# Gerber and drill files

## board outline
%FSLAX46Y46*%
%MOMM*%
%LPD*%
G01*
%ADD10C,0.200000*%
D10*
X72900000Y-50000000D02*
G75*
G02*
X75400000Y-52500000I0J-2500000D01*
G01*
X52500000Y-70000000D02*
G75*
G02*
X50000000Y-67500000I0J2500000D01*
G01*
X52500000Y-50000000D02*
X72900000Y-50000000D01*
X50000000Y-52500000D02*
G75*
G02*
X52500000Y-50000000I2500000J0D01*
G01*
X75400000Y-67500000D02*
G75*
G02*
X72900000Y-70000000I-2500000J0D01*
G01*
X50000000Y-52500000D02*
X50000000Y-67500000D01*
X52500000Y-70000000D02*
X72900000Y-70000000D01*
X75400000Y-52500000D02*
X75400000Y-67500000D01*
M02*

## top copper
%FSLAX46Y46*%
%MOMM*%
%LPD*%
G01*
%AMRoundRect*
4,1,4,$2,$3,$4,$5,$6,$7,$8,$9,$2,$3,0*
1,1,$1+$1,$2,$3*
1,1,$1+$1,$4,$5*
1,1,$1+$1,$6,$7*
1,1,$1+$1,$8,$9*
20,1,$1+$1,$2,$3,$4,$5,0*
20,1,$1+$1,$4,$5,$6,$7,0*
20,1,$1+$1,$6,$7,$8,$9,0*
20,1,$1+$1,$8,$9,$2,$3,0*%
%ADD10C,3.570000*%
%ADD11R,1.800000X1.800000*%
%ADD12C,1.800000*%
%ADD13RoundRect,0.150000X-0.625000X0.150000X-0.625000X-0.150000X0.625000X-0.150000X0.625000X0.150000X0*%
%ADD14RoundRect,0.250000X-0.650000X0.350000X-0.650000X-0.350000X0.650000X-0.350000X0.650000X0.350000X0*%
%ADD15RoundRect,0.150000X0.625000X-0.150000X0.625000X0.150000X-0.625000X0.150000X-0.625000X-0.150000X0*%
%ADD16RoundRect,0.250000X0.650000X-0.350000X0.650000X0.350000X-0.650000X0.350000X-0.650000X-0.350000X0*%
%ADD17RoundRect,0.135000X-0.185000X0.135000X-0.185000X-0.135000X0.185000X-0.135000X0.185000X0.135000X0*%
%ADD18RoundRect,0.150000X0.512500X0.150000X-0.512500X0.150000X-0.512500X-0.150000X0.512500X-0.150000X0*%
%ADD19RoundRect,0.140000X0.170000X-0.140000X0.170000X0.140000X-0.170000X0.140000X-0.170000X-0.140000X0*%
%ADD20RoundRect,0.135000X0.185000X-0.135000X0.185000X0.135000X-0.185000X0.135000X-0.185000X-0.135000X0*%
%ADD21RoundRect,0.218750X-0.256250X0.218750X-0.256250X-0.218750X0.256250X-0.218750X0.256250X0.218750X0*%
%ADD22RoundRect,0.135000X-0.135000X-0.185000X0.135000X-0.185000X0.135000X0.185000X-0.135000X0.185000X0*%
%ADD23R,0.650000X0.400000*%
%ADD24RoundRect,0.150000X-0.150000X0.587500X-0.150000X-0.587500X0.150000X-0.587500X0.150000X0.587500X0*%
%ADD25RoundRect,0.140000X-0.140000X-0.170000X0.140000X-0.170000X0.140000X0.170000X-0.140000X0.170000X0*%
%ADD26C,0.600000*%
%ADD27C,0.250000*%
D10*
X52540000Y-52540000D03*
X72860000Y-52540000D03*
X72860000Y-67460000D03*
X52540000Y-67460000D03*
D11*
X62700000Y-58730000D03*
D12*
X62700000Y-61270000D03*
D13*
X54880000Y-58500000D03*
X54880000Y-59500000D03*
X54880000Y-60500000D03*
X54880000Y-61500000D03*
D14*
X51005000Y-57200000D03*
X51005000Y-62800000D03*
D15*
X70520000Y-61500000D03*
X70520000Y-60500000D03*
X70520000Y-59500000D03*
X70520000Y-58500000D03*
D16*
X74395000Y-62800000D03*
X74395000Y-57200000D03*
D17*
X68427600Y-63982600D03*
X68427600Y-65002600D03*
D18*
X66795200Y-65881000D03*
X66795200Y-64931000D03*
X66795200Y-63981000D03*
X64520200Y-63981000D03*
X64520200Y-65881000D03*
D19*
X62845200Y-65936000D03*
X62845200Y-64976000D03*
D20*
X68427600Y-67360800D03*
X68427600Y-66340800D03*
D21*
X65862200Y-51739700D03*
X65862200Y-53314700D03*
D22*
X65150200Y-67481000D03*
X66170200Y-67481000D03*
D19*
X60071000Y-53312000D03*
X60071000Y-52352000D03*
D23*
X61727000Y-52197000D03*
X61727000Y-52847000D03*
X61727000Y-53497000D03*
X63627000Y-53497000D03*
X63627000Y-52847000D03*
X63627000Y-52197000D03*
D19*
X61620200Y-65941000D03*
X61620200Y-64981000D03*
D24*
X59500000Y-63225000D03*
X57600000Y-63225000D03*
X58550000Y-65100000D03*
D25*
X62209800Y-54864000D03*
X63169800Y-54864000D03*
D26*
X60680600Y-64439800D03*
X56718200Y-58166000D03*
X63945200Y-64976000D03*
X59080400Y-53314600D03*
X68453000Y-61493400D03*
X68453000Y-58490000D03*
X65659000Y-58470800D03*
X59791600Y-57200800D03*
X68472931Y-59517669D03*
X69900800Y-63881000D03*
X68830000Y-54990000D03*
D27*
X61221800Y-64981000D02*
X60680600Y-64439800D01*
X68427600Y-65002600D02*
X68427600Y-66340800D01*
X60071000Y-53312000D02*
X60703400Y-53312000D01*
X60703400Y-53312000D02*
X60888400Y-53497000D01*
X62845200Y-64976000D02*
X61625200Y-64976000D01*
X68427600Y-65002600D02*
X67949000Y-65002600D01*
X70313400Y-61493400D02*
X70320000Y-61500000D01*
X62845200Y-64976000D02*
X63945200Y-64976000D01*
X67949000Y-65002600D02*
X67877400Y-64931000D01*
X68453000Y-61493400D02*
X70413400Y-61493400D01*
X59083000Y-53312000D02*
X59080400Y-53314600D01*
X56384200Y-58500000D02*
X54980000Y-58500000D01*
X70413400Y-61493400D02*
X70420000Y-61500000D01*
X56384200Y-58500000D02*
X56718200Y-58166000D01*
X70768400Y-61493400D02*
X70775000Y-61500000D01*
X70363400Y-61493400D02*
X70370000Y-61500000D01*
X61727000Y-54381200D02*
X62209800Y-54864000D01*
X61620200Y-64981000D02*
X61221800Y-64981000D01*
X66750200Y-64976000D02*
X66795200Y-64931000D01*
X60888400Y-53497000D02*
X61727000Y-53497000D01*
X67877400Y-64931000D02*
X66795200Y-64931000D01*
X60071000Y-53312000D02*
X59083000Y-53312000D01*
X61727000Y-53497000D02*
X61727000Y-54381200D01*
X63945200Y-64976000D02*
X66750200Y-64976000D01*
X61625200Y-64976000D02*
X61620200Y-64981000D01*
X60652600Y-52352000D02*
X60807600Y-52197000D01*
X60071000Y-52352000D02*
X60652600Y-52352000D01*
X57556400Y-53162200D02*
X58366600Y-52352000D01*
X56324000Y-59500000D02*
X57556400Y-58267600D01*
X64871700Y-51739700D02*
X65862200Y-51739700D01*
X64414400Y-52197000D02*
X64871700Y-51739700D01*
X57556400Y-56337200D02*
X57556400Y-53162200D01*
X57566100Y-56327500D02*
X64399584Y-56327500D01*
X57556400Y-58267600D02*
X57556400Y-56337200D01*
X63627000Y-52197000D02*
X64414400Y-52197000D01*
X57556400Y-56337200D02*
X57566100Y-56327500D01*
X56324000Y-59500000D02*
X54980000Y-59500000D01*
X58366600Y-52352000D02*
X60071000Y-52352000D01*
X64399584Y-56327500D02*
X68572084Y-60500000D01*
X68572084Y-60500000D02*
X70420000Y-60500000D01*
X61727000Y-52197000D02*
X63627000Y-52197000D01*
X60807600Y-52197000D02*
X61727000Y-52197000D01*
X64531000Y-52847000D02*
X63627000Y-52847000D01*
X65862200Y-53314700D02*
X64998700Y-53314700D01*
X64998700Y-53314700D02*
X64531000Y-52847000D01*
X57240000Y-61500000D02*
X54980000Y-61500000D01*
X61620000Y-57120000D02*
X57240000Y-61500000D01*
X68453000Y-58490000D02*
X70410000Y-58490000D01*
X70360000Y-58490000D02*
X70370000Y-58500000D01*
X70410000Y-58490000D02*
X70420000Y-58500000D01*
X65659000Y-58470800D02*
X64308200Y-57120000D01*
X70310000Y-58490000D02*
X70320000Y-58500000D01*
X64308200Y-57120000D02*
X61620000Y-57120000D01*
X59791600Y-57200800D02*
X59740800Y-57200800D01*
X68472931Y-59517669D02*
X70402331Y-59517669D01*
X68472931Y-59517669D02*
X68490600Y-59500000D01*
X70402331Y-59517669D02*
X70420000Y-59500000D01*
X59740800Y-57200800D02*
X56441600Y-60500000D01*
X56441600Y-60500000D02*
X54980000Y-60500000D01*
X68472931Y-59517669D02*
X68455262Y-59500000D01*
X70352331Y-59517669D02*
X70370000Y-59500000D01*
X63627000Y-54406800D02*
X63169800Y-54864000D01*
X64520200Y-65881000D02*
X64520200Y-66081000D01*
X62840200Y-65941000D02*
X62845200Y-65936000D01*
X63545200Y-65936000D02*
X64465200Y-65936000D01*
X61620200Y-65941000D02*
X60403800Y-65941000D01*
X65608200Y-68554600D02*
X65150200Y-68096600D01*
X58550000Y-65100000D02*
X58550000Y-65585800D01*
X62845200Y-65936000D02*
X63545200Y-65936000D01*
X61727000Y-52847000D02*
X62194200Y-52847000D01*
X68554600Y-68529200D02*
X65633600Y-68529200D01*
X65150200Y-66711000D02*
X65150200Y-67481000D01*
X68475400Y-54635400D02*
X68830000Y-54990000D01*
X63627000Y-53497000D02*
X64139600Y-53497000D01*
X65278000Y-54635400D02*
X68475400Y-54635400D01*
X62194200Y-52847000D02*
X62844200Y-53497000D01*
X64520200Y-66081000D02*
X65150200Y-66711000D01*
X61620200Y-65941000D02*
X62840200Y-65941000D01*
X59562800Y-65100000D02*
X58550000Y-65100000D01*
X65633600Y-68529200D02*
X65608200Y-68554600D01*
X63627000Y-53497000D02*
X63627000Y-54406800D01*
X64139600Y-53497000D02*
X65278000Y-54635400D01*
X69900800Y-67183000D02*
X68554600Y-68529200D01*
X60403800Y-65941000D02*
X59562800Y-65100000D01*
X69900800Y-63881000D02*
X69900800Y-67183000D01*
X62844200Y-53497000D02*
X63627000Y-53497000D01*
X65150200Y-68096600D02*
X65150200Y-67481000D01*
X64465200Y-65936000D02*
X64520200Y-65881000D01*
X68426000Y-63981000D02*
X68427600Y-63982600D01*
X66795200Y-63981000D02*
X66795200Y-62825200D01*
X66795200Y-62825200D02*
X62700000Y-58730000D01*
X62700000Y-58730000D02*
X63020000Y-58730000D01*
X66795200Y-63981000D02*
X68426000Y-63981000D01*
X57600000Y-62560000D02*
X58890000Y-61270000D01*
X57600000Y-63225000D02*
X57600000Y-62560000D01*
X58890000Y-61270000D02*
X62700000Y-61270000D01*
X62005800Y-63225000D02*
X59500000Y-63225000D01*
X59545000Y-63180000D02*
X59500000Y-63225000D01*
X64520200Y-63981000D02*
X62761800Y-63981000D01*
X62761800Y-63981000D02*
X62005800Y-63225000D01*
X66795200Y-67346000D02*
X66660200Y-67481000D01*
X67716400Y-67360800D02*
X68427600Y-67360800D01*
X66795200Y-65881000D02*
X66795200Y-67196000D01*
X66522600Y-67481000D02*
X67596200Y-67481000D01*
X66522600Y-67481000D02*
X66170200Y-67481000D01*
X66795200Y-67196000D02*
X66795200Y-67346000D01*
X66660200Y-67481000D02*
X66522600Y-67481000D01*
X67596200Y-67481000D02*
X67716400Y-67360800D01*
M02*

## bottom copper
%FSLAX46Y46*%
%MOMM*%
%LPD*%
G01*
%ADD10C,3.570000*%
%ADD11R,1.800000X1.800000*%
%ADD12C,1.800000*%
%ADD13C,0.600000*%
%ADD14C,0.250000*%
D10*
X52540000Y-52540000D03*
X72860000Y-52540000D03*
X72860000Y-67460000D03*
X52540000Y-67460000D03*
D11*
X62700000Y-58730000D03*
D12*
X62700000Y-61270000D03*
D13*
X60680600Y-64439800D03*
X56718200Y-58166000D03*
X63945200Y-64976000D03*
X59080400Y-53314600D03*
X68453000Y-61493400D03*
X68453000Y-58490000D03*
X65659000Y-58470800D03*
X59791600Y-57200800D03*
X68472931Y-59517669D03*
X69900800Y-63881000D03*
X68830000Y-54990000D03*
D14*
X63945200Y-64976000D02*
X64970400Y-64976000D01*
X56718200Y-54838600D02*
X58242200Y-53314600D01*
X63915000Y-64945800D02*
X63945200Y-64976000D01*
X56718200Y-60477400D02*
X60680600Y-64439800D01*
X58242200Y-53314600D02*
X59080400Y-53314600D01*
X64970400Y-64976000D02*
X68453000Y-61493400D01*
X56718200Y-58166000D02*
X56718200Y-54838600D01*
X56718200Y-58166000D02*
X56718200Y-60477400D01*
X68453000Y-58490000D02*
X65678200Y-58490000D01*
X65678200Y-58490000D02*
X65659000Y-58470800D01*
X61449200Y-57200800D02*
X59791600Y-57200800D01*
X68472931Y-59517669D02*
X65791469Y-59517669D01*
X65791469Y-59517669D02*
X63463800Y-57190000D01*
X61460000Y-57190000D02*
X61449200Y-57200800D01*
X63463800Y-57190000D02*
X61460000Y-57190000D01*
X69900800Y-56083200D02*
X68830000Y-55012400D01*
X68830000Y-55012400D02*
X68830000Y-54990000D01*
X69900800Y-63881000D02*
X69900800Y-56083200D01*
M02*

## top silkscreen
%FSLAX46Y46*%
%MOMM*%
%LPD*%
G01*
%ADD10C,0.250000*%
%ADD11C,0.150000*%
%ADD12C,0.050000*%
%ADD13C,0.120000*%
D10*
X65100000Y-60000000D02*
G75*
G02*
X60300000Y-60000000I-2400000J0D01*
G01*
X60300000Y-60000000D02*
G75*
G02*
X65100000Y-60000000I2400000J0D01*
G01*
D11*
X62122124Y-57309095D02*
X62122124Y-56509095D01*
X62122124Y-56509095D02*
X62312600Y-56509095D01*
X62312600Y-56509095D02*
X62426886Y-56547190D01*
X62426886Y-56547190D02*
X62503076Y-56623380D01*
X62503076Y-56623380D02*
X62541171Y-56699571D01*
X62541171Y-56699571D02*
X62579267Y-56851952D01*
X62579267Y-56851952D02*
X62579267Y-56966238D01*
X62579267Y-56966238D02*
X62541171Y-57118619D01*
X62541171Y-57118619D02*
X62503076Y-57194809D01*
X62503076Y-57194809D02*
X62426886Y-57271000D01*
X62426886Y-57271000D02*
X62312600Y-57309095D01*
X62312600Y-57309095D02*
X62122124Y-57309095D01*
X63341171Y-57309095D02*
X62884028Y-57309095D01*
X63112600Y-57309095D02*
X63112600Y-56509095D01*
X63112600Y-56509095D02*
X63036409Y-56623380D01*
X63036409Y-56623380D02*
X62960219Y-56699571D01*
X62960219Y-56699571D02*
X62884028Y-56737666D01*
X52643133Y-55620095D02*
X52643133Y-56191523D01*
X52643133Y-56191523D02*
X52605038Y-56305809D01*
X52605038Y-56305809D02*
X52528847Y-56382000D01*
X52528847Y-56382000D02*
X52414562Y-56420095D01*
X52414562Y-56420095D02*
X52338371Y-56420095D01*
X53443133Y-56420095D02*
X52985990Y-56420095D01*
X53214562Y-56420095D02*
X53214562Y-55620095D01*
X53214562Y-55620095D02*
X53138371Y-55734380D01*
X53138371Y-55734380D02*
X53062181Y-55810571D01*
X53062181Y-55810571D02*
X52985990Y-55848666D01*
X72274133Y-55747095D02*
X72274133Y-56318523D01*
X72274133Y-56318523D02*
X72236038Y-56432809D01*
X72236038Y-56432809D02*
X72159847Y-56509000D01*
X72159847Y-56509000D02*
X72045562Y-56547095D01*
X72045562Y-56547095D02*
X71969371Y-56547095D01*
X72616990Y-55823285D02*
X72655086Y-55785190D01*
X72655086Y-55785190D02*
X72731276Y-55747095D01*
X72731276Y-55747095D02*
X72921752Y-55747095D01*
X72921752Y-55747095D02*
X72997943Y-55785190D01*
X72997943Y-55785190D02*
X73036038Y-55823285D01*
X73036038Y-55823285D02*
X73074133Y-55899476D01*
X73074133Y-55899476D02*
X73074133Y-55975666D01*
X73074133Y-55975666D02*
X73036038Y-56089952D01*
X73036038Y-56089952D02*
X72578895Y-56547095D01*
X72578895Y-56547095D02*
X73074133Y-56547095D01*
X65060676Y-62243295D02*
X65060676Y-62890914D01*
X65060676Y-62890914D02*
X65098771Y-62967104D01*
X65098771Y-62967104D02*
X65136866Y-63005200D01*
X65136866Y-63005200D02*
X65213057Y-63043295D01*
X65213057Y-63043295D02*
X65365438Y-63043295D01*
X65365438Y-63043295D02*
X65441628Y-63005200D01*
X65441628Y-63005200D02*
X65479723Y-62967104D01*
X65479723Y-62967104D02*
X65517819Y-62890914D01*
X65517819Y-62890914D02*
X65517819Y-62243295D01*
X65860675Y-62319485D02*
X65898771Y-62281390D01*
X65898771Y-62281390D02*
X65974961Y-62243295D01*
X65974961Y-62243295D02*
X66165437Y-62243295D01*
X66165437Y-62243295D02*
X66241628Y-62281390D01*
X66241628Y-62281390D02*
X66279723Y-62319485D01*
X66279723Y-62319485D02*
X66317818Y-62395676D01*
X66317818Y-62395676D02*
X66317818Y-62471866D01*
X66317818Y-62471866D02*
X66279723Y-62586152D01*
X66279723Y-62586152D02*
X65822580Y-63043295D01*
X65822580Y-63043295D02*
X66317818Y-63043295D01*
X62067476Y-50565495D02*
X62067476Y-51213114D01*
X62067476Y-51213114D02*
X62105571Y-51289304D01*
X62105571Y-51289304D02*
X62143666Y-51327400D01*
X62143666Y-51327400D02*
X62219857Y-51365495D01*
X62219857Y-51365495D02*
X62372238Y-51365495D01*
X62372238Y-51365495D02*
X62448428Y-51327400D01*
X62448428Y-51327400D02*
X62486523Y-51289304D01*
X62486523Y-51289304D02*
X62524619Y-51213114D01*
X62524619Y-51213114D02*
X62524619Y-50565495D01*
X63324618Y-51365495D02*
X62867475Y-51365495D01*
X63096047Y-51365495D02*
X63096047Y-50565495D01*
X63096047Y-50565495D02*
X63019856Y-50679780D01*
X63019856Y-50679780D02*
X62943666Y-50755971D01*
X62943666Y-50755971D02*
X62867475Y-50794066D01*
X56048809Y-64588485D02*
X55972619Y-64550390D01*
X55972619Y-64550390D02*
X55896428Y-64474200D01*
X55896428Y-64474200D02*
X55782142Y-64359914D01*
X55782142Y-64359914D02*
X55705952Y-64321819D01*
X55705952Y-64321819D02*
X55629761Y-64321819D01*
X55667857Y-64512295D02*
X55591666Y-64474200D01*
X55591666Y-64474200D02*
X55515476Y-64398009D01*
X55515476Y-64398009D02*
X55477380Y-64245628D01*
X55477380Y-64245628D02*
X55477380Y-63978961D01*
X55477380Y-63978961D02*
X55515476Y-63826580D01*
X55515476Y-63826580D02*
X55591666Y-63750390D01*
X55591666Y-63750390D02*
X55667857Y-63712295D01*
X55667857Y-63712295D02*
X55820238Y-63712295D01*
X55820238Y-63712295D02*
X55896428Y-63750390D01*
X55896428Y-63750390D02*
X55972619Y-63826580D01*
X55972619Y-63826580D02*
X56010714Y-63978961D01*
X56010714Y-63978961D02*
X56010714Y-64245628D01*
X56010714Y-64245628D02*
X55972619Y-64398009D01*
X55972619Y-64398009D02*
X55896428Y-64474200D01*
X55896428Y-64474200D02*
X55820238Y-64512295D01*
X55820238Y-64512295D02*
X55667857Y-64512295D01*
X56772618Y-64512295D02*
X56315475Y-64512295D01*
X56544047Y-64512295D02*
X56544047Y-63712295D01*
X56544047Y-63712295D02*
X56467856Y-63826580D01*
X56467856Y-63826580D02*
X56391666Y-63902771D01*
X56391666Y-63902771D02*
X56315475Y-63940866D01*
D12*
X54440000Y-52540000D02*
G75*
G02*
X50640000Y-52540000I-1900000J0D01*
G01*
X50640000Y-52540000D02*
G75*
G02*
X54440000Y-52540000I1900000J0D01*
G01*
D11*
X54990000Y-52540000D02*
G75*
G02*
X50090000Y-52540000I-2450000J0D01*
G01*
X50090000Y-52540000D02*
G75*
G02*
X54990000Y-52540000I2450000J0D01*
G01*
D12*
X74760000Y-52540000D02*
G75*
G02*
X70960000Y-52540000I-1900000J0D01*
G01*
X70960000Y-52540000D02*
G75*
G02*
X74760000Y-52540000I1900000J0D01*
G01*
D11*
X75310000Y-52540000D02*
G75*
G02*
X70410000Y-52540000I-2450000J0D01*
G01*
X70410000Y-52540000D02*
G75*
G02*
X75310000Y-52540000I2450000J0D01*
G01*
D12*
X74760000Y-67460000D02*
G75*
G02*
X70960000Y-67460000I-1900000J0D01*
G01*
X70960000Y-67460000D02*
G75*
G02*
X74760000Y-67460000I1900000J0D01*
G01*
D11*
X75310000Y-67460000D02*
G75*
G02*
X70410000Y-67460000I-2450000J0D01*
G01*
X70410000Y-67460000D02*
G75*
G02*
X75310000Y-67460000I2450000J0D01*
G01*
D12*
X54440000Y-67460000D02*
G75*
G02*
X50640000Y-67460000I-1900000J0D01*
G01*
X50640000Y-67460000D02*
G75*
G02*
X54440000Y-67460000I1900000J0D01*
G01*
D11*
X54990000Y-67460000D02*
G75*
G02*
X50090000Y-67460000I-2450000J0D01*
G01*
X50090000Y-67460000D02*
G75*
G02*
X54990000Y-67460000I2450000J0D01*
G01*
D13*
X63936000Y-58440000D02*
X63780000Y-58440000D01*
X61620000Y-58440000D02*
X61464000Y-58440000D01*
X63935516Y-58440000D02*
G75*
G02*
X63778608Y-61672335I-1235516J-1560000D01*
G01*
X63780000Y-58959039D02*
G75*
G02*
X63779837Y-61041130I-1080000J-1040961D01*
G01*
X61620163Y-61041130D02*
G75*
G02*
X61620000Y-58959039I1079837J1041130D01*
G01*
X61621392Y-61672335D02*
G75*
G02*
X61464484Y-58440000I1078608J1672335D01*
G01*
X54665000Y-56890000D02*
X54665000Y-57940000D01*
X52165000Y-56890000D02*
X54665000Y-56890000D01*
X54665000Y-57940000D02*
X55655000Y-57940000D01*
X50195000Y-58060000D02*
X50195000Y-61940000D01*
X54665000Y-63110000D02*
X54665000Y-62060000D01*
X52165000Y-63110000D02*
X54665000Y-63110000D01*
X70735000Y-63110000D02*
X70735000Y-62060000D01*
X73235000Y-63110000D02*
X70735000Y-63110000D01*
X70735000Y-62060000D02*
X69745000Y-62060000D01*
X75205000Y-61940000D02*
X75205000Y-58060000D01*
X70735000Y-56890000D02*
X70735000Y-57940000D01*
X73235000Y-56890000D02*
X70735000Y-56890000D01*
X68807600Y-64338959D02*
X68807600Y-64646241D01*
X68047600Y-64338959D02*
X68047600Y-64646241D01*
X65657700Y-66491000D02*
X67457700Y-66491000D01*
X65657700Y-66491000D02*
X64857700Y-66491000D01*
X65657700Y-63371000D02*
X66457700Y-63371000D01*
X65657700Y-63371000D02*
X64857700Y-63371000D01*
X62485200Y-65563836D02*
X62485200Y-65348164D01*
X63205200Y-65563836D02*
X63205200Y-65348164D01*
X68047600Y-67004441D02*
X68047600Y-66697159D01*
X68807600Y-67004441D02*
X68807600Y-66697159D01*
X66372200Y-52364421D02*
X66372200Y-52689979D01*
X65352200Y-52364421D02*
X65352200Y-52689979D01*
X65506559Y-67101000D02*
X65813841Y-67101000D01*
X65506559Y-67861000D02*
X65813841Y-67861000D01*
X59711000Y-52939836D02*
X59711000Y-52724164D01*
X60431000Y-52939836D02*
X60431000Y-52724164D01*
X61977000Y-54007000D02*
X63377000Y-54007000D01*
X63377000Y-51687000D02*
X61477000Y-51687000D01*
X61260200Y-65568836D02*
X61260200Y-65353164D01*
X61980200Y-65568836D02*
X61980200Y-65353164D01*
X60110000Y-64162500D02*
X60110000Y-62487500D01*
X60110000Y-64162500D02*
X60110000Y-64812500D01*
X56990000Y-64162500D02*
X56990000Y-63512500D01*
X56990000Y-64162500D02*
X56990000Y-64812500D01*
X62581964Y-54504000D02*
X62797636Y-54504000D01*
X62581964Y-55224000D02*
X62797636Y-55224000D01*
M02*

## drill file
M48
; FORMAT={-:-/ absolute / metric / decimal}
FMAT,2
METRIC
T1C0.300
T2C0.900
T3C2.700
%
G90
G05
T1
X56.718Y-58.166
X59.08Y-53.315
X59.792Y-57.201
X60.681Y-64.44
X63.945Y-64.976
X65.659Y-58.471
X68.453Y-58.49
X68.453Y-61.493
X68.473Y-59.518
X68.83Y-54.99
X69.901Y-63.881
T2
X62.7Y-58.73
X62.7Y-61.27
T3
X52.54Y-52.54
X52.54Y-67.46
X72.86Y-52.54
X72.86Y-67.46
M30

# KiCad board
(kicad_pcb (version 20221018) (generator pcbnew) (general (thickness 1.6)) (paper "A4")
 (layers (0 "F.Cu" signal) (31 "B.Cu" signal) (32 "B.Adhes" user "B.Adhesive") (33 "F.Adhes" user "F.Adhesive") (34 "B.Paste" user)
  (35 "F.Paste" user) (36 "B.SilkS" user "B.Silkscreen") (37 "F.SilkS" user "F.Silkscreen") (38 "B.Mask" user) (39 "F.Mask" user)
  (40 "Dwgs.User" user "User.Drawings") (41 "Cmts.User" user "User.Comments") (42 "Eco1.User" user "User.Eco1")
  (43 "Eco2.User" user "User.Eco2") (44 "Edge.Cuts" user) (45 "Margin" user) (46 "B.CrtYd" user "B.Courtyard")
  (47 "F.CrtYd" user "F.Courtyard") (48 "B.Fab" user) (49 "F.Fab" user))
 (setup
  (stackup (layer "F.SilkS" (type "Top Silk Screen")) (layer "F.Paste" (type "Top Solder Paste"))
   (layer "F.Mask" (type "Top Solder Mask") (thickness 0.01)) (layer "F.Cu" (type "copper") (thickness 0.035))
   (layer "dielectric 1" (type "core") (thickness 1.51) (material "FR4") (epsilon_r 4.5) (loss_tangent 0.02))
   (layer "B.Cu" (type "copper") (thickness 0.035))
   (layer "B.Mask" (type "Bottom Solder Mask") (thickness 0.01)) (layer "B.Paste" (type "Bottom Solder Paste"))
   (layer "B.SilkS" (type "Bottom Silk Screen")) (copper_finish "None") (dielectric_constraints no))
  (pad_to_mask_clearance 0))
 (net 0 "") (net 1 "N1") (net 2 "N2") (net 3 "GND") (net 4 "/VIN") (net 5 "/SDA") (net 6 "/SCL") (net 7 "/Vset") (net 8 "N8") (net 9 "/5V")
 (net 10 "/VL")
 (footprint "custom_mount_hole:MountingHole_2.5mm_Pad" (layer "F.Cu") (at 52.54 52.54)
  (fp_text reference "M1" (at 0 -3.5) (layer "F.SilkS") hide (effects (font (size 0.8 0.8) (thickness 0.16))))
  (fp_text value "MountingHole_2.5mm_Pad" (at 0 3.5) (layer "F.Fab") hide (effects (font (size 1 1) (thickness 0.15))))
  (fp_circle (center 0 0) (end 1.9 0) (stroke (width 0.05) (type solid)) (fill none) (layer "F.SilkS"))
  (fp_circle (center 0 0) (end 2.45 0) (stroke (width 0.15) (type solid)) (fill none) (layer "F.SilkS"))
  (pad "~" thru_hole circle (at 0 0) (size 3.57 3.57) (drill 2.7) (layers "*.Cu" "*.Mask")))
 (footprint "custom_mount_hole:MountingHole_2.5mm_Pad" (layer "F.Cu") (at 72.86 52.54)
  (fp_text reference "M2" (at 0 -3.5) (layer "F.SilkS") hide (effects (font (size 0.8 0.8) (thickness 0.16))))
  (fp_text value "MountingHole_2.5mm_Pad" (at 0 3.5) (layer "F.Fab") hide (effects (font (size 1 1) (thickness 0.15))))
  (fp_circle (center 0 0) (end 1.9 0) (stroke (width 0.05) (type solid)) (fill none) (layer "F.SilkS"))
  (fp_circle (center 0 0) (end 2.45 0) (stroke (width 0.15) (type solid)) (fill none) (layer "F.SilkS"))
  (pad "~" thru_hole circle (at 0 0) (size 3.57 3.57) (drill 2.7) (layers "*.Cu" "*.Mask")))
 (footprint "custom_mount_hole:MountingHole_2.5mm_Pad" (layer "F.Cu") (at 72.86 67.46)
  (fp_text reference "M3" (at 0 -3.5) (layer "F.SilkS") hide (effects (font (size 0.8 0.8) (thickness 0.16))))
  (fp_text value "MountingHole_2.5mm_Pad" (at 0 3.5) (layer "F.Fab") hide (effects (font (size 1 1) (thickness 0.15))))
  (fp_circle (center 0 0) (end 1.9 0) (stroke (width 0.05) (type solid)) (fill none) (layer "F.SilkS"))
  (fp_circle (center 0 0) (end 2.45 0) (stroke (width 0.15) (type solid)) (fill none) (layer "F.SilkS"))
  (pad "~" thru_hole circle (at 0 0) (size 3.57 3.57) (drill 2.7) (layers "*.Cu" "*.Mask")))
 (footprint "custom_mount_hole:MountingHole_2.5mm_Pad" (layer "F.Cu") (at 52.54 67.46)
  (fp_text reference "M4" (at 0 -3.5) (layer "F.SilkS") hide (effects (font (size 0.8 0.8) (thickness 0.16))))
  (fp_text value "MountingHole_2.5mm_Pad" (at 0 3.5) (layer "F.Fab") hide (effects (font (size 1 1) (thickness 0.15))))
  (fp_circle (center 0 0) (end 1.9 0) (stroke (width 0.05) (type solid)) (fill none) (layer "F.SilkS"))
  (fp_circle (center 0 0) (end 2.45 0) (stroke (width 0.15) (type solid)) (fill none) (layer "F.SilkS"))
  (pad "~" thru_hole circle (at 0 0) (size 3.57 3.57) (drill 2.7) (layers "*.Cu" "*.Mask")))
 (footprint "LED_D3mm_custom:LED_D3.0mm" (layer "F.Cu") (at 62.7 58.73 -90)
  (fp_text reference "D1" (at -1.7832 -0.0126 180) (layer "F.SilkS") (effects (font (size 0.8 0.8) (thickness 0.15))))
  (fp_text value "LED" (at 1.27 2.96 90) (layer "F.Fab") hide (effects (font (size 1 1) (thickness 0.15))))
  (fp_line (start -0.29 -1.236) (end -0.29 -1.08) (stroke (width 0.12) (type solid)) (layer "F.SilkS"))
  (fp_line (start -0.29 1.08) (end -0.29 1.236) (stroke (width 0.12) (type solid)) (layer "F.SilkS"))
  (fp_arc (start -0.29 -1.235516) (mid 1.366487 -1.987659) (end 2.942335 -1.078608) (stroke (width 0.12) (type solid)) (layer "F.SilkS"))
  (fp_arc (start 0.229039 -1.08) (mid 1.270117 -1.5) (end 2.31113 -1.079837) (stroke (width 0.12) (type solid)) (layer "F.SilkS"))
  (fp_arc (start 2.31113 1.079837) (mid 1.270117 1.5) (end 0.229039 1.08) (stroke (width 0.12) (type solid)) (layer "F.SilkS"))
  (fp_arc (start 2.942335 1.078608) (mid 1.366487 1.987659) (end -0.29 1.235516) (stroke (width 0.12) (type solid)) (layer "F.SilkS"))
  (pad "1" thru_hole rect (at 0 0 270) (size 1.8 1.8) (drill 0.9) (layers "*.Cu" "*.Mask") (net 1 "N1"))
  (pad "2" thru_hole circle (at 2.54 0 270) (size 1.8 1.8) (drill 0.9) (layers "*.Cu" "*.Mask") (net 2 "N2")))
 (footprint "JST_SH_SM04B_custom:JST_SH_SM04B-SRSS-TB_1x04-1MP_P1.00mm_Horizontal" (layer "F.Cu") (at 52.88 60 -90)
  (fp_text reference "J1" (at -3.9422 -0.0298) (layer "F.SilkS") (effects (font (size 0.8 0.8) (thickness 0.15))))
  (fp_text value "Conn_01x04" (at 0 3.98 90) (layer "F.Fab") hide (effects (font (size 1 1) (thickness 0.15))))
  (fp_line (start -3.11 -1.785) (end -2.06 -1.785) (stroke (width 0.12) (type solid)) (layer "F.SilkS"))
  (fp_line (start -3.11 0.715) (end -3.11 -1.785) (stroke (width 0.12) (type solid)) (layer "F.SilkS"))
  (fp_line (start -2.06 -1.785) (end -2.06 -2.775) (stroke (width 0.12) (type solid)) (layer "F.SilkS"))
  (fp_line (start -1.94 2.685) (end 1.94 2.685) (stroke (width 0.12) (type solid)) (layer "F.SilkS"))
  (fp_line (start 3.11 -1.785) (end 2.06 -1.785) (stroke (width 0.12) (type solid)) (layer "F.SilkS"))
  (fp_line (start 3.11 0.715) (end 3.11 -1.785) (stroke (width 0.12) (type solid)) (layer "F.SilkS"))
  (pad "1" smd roundrect (at -1.5 -2 270) (size 0.6 1.55) (layers "F.Cu" "F.Paste" "F.Mask") (roundrect_rratio 0.25) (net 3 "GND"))
  (pad "2" smd roundrect (at -0.5 -2 270) (size 0.6 1.55) (layers "F.Cu" "F.Paste" "F.Mask") (roundrect_rratio 0.25) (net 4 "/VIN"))
  (pad "3" smd roundrect (at 0.5 -2 270) (size 0.6 1.55) (layers "F.Cu" "F.Paste" "F.Mask") (roundrect_rratio 0.25) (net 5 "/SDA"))
  (pad "4" smd roundrect (at 1.5 -2 270) (size 0.6 1.55) (layers "F.Cu" "F.Paste" "F.Mask") (roundrect_rratio 0.25) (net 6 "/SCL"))
  (pad "MP" smd roundrect (at -2.8 1.875 270) (size 1.2 1.8) (layers "F.Cu" "F.Paste" "F.Mask") (roundrect_rratio 0.2083333333))
  (pad "MP" smd roundrect (at 2.8 1.875 270) (size 1.2 1.8) (layers "F.Cu" "F.Paste" "F.Mask") (roundrect_rratio 0.2083333333)))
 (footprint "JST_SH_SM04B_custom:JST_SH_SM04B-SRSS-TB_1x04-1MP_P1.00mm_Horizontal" (layer "F.Cu") (at 72.52 60 90)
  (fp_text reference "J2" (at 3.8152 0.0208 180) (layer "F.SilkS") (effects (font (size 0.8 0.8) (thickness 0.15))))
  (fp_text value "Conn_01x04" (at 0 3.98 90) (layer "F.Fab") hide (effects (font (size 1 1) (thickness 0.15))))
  (fp_line (start -3.11 -1.785) (end -2.06 -1.785) (stroke (width 0.12) (type solid)) (layer "F.SilkS"))
  (fp_line (start -3.11 0.715) (end -3.11 -1.785) (stroke (width 0.12) (type solid)) (layer "F.SilkS"))
  (fp_line (start -2.06 -1.785) (end -2.06 -2.775) (stroke (width 0.12) (type solid)) (layer "F.SilkS"))
  (fp_line (start -1.94 2.685) (end 1.94 2.685) (stroke (width 0.12) (type solid)) (layer "F.SilkS"))
  (fp_line (start 3.11 -1.785) (end 2.06 -1.785) (stroke (width 0.12) (type solid)) (layer "F.SilkS"))
  (fp_line (start 3.11 0.715) (end 3.11 -1.785) (stroke (width 0.12) (type solid)) (layer "F.SilkS"))
  (pad "1" smd roundrect (at -1.5 -2 90) (size 0.6 1.55) (layers "F.Cu" "F.Paste" "F.Mask") (roundrect_rratio 0.25) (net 3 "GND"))
  (pad "2" smd roundrect (at -0.5 -2 90) (size 0.6 1.55) (layers "F.Cu" "F.Paste" "F.Mask") (roundrect_rratio 0.25) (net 4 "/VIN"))
  (pad "3" smd roundrect (at 0.5 -2 90) (size 0.6 1.55) (layers "F.Cu" "F.Paste" "F.Mask") (roundrect_rratio 0.25) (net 5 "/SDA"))
  (pad "4" smd roundrect (at 1.5 -2 90) (size 0.6 1.55) (layers "F.Cu" "F.Paste" "F.Mask") (roundrect_rratio 0.25) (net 6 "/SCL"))
  (pad "MP" smd roundrect (at -2.8 1.875 90) (size 1.2 1.8) (layers "F.Cu" "F.Paste" "F.Mask") (roundrect_rratio 0.2083333333))
  (pad "MP" smd roundrect (at 2.8 1.875 90) (size 1.2 1.8) (layers "F.Cu" "F.Paste" "F.Mask") (roundrect_rratio 0.2083333333)))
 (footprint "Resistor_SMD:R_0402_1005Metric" (layer "F.Cu") (at 68.4276 64.4926 -90)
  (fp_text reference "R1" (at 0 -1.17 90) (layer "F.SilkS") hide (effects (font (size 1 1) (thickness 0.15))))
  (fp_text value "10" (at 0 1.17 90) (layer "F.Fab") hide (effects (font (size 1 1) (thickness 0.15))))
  (fp_line (start -0.153641 -0.38) (end 0.153641 -0.38) (stroke (width 0.12) (type solid)) (layer "F.SilkS"))
  (fp_line (start -0.153641 0.38) (end 0.153641 0.38) (stroke (width 0.12) (type solid)) (layer "F.SilkS"))
  (pad "1" smd roundrect (at -0.51 0 270) (size 0.54 0.64) (layers "F.Cu" "F.Paste" "F.Mask") (roundrect_rratio 0.25) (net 1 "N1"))
  (pad "2" smd roundrect (at 0.51 0 270) (size 0.54 0.64) (layers "F.Cu" "F.Paste" "F.Mask") (roundrect_rratio 0.25) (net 3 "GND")))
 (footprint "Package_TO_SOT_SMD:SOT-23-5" (layer "F.Cu") (at 65.6577 64.931 180)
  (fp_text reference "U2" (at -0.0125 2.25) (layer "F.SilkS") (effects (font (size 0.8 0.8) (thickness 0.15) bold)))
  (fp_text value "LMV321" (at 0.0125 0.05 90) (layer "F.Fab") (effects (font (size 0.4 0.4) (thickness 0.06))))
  (fp_line (start 0 -1.56) (end -1.8 -1.56) (stroke (width 0.12) (type solid)) (layer "F.SilkS"))
  (fp_line (start 0 -1.56) (end 0.8 -1.56) (stroke (width 0.12) (type solid)) (layer "F.SilkS"))
  (fp_line (start 0 1.56) (end -0.8 1.56) (stroke (width 0.12) (type solid)) (layer "F.SilkS"))
  (fp_line (start 0 1.56) (end 0.8 1.56) (stroke (width 0.12) (type solid)) (layer "F.SilkS"))
  (pad "1" smd roundrect (at -1.1375 -0.95 180) (size 1.325 0.6) (layers "F.Cu" "F.Paste" "F.Mask") (roundrect_rratio 0.25) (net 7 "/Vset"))
  (pad "2" smd roundrect (at -1.1375 0 180) (size 1.325 0.6) (layers "F.Cu" "F.Paste" "F.Mask") (roundrect_rratio 0.25) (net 3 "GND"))
  (pad "3" smd roundrect (at -1.1375 0.95 180) (size 1.325 0.6) (layers "F.Cu" "F.Paste" "F.Mask") (roundrect_rratio 0.25) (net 1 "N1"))
  (pad "4" smd roundrect (at 1.1375 0.95 180) (size 1.325 0.6) (layers "F.Cu" "F.Paste" "F.Mask") (roundrect_rratio 0.25) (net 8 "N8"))
  (pad "5" smd roundrect (at 1.1375 -0.95 180) (size 1.325 0.6) (layers "F.Cu" "F.Paste" "F.Mask") (roundrect_rratio 0.25) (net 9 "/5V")))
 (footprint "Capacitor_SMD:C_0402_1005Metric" (layer "F.Cu") (at 62.8452 65.456 90)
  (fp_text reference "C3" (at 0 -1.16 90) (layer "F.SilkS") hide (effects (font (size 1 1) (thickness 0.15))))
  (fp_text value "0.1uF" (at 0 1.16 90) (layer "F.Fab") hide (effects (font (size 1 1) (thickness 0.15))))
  (fp_line (start -0.107836 -0.36) (end 0.107836 -0.36) (stroke (width 0.12) (type solid)) (layer "F.SilkS"))
  (fp_line (start -0.107836 0.36) (end 0.107836 0.36) (stroke (width 0.12) (type solid)) (layer "F.SilkS"))
  (pad "1" smd roundrect (at -0.48 0 90) (size 0.56 0.62) (layers "F.Cu" "F.Paste" "F.Mask") (roundrect_rratio 0.25) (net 9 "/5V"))
  (pad "2" smd roundrect (at 0.48 0 90) (size 0.56 0.62) (layers "F.Cu" "F.Paste" "F.Mask") (roundrect_rratio 0.25) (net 3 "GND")))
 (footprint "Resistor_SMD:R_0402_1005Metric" (layer "F.Cu") (at 68.4276 66.8508 90)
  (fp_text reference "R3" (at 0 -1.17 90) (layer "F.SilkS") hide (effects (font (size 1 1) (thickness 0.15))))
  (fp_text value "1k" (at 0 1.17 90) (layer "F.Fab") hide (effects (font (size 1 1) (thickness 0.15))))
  (fp_line (start -0.153641 -0.38) (end 0.153641 -0.38) (stroke (width 0.12) (type solid)) (layer "F.SilkS"))
  (fp_line (start -0.153641 0.38) (end 0.153641 0.38) (stroke (width 0.12) (type solid)) (layer "F.SilkS"))
  (pad "1" smd roundrect (at -0.51 0 90) (size 0.54 0.64) (layers "F.Cu" "F.Paste" "F.Mask") (roundrect_rratio 0.25) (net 7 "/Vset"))
  (pad "2" smd roundrect (at 0.51 0 90) (size 0.54 0.64) (layers "F.Cu" "F.Paste" "F.Mask") (roundrect_rratio 0.25) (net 3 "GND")))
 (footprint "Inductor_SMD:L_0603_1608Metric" (layer "F.Cu") (at 65.8622 52.5272 -90)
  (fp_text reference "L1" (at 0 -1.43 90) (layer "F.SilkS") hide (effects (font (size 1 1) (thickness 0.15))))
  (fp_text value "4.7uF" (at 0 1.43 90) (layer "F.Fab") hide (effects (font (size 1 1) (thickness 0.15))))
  (fp_line (start -0.162779 -0.51) (end 0.162779 -0.51) (stroke (width 0.12) (type solid)) (layer "F.SilkS"))
  (fp_line (start -0.162779 0.51) (end 0.162779 0.51) (stroke (width 0.12) (type solid)) (layer "F.SilkS"))
  (pad "1" smd roundrect (at -0.7875 0 270) (size 0.875 0.95) (layers "F.Cu" "F.Paste" "F.Mask") (roundrect_rratio 0.25) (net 4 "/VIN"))
  (pad "2" smd roundrect (at 0.7875 0 270) (size 0.875 0.95) (layers "F.Cu" "F.Paste" "F.Mask") (roundrect_rratio 0.25) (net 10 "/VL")))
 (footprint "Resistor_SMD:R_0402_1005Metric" (layer "F.Cu") (at 65.6602 67.481)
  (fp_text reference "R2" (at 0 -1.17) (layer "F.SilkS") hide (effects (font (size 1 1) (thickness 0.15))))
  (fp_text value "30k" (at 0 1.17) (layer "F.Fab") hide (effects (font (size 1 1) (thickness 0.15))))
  (fp_line (start -0.153641 -0.38) (end 0.153641 -0.38) (stroke (width 0.12) (type solid)) (layer "F.SilkS"))
  (fp_line (start -0.153641 0.38) (end 0.153641 0.38) (stroke (width 0.12) (type solid)) (layer "F.SilkS"))
  (pad "1" smd roundrect (at -0.51 0) (size 0.54 0.64) (layers "F.Cu" "F.Paste" "F.Mask") (roundrect_rratio 0.25) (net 9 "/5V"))
  (pad "2" smd roundrect (at 0.51 0) (size 0.54 0.64) (layers "F.Cu" "F.Paste" "F.Mask") (roundrect_rratio 0.25) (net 7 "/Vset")))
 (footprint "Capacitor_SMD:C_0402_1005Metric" (layer "F.Cu") (at 60.071 52.832 90)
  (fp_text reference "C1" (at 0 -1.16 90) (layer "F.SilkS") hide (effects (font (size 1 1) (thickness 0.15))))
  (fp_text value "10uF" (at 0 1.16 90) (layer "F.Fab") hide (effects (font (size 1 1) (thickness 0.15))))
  (fp_line (start -0.107836 -0.36) (end 0.107836 -0.36) (stroke (width 0.12) (type solid)) (layer "F.SilkS"))
  (fp_line (start -0.107836 0.36) (end 0.107836 0.36) (stroke (width 0.12) (type solid)) (layer "F.SilkS"))
  (pad "1" smd roundrect (at -0.48 0 90) (size 0.56 0.62) (layers "F.Cu" "F.Paste" "F.Mask") (roundrect_rratio 0.25) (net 3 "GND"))
  (pad "2" smd roundrect (at 0.48 0 90) (size 0.56 0.62) (layers "F.Cu" "F.Paste" "F.Mask") (roundrect_rratio 0.25) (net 4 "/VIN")))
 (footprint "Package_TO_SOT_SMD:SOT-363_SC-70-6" (layer "F.Cu") (at 62.677 52.847)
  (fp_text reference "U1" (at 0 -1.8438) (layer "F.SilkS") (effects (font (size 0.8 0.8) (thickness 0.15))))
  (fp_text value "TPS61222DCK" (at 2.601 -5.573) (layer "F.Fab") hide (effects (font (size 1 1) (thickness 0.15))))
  (fp_line (start -0.7 1.16) (end 0.7 1.16) (stroke (width 0.12) (type solid)) (layer "F.SilkS"))
  (fp_line (start 0.7 -1.16) (end -1.2 -1.16) (stroke (width 0.12) (type solid)) (layer "F.SilkS"))
  (pad "1" smd rect (at -0.95 -0.65) (size 0.65 0.4) (layers "F.Cu" "F.Paste" "F.Mask") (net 4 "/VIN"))
  (pad "2" smd rect (at -0.95 0) (size 0.65 0.4) (layers "F.Cu" "F.Paste" "F.Mask") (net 9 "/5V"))
  (pad "3" smd rect (at -0.95 0.65) (size 0.65 0.4) (layers "F.Cu" "F.Paste" "F.Mask") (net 3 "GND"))
  (pad "4" smd rect (at 0.95 0.65) (size 0.65 0.4) (layers "F.Cu" "F.Paste" "F.Mask") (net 9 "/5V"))
  (pad "5" smd rect (at 0.95 0) (size 0.65 0.4) (layers "F.Cu" "F.Paste" "F.Mask") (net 10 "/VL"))
  (pad "6" smd rect (at 0.95 -0.65) (size 0.65 0.4) (layers "F.Cu" "F.Paste" "F.Mask") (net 4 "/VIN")))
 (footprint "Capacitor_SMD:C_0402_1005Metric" (layer "F.Cu") (at 61.6202 65.461 90)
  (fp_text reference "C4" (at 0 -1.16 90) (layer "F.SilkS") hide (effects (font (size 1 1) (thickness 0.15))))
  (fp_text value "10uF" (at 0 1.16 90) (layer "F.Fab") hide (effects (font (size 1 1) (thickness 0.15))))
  (fp_line (start -0.107836 -0.36) (end 0.107836 -0.36) (stroke (width 0.12) (type solid)) (layer "F.SilkS"))
  (fp_line (start -0.107836 0.36) (end 0.107836 0.36) (stroke (width 0.12) (type solid)) (layer "F.SilkS"))
  (pad "1" smd roundrect (at -0.48 0 90) (size 0.56 0.62) (layers "F.Cu" "F.Paste" "F.Mask") (roundrect_rratio 0.25) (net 9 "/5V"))
  (pad "2" smd roundrect (at 0.48 0 90) (size 0.56 0.62) (layers "F.Cu" "F.Paste" "F.Mask") (roundrect_rratio 0.25) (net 3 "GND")))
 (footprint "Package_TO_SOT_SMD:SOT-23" (layer "F.Cu") (at 58.55 64.1625 -90)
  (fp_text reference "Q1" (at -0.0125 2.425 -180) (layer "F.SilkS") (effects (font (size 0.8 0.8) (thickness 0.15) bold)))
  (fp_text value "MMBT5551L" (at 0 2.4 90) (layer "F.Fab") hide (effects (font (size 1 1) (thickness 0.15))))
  (fp_line (start 0 -1.56) (end -1.675 -1.56) (stroke (width 0.12) (type solid)) (layer "F.SilkS"))
  (fp_line (start 0 -1.56) (end 0.65 -1.56) (stroke (width 0.12) (type solid)) (layer "F.SilkS"))
  (fp_line (start 0 1.56) (end -0.65 1.56) (stroke (width 0.12) (type solid)) (layer "F.SilkS"))
  (fp_line (start 0 1.56) (end 0.65 1.56) (stroke (width 0.12) (type solid)) (layer "F.SilkS"))
  (pad "1" smd roundrect (at -0.9375 -0.95 270) (size 1.475 0.6) (layers "F.Cu" "F.Paste" "F.Mask") (roundrect_rratio 0.25) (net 8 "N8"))
  (pad "2" smd roundrect (at -0.9375 0.95 270) (size 1.475 0.6) (layers "F.Cu" "F.Paste" "F.Mask") (roundrect_rratio 0.25) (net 2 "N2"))
  (pad "3" smd roundrect (at 0.9375 0 270) (size 1.475 0.6) (layers "F.Cu" "F.Paste" "F.Mask") (roundrect_rratio 0.25) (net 9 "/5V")))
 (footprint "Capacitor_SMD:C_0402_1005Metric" (layer "F.Cu") (at 62.6898 54.864)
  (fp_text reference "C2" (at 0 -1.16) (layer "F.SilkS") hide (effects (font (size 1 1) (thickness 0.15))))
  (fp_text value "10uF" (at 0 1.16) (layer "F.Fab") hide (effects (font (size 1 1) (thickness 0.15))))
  (fp_line (start -0.107836 -0.36) (end 0.107836 -0.36) (stroke (width 0.12) (type solid)) (layer "F.SilkS"))
  (fp_line (start -0.107836 0.36) (end 0.107836 0.36) (stroke (width 0.12) (type solid)) (layer "F.SilkS"))
  (pad "1" smd roundrect (at -0.48 0) (size 0.56 0.62) (layers "F.Cu" "F.Paste" "F.Mask") (roundrect_rratio 0.25) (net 3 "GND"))
  (pad "2" smd roundrect (at 0.48 0) (size 0.56 0.62) (layers "F.Cu" "F.Paste" "F.Mask") (roundrect_rratio 0.25) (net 9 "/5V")))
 (gr_circle (center 62.7 60) (end 65.1 60) (stroke (width 0.25) (type solid)) (fill none) (layer "F.SilkS"))
 (gr_arc (start 72.9 50) (mid 74.667767 50.732233) (end 75.4 52.5) (stroke (width 0.2) (type solid)) (layer "Edge.Cuts"))
 (gr_arc (start 52.5 70) (mid 50.732233 69.267767) (end 50 67.5) (stroke (width 0.2) (type solid)) (layer "Edge.Cuts"))
 (gr_line (start 52.5 50) (end 72.9 50) (stroke (width 0.2) (type solid)) (layer "Edge.Cuts"))
 (gr_arc (start 50 52.5) (mid 50.732233 50.732233) (end 52.5 50) (stroke (width 0.2) (type solid)) (layer "Edge.Cuts"))
 (gr_arc (start 75.4 67.5) (mid 74.667767 69.267767) (end 72.9 70) (stroke (width 0.2) (type solid)) (layer "Edge.Cuts"))
 (gr_line (start 50 52.5) (end 50 67.5) (stroke (width 0.2) (type solid)) (layer "Edge.Cuts"))
 (gr_line (start 52.5 70) (end 72.9 70) (stroke (width 0.2) (type solid)) (layer "Edge.Cuts"))
 (gr_line (start 75.4 52.5) (end 75.4 67.5) (stroke (width 0.2) (type solid)) (layer "Edge.Cuts"))
 (segment (start 61.2218 64.981) (end 60.6806 64.4398) (width 0.25) (layer "F.Cu") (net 3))
 (segment (start 68.4276 65.0026) (end 68.4276 66.3408) (width 0.25) (layer "F.Cu") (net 3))
 (segment (start 60.071 53.312) (end 60.7034 53.312) (width 0.25) (layer "F.Cu") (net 3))
 (segment (start 60.7034 53.312) (end 60.8884 53.497) (width 0.25) (layer "F.Cu") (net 3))
 (segment (start 62.8452 64.976) (end 61.6252 64.976) (width 0.25) (layer "F.Cu") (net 3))
 (segment (start 68.4276 65.0026) (end 67.949 65.0026) (width 0.25) (layer "F.Cu") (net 3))
 (segment (start 70.3134 61.4934) (end 70.32 61.5) (width 0.25) (layer "F.Cu") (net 3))
 (segment (start 62.8452 64.976) (end 63.9452 64.976) (width 0.25) (layer "F.Cu") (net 3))
 (segment (start 67.949 65.0026) (end 67.8774 64.931) (width 0.25) (layer "F.Cu") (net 3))
 (segment (start 68.453 61.4934) (end 70.4134 61.4934) (width 0.25) (layer "F.Cu") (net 3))
 (segment (start 59.083 53.312) (end 59.0804 53.3146) (width 0.25) (layer "F.Cu") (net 3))
 (segment (start 56.3842 58.5) (end 54.98 58.5) (width 0.25) (layer "F.Cu") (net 3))
 (segment (start 70.4134 61.4934) (end 70.42 61.5) (width 0.25) (layer "F.Cu") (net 3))
 (segment (start 56.3842 58.5) (end 56.7182 58.166) (width 0.25) (layer "F.Cu") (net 3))
 (segment (start 70.7684 61.4934) (end 70.775 61.5) (width 0.25) (layer "F.Cu") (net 3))
 (segment (start 70.3634 61.4934) (end 70.37 61.5) (width 0.25) (layer "F.Cu") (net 3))
 (segment (start 61.727 54.3812) (end 62.2098 54.864) (width 0.25) (layer "F.Cu") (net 3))
 (segment (start 61.6202 64.981) (end 61.2218 64.981) (width 0.25) (layer "F.Cu") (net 3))
 (segment (start 66.7502 64.976) (end 66.7952 64.931) (width 0.25) (layer "F.Cu") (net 3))
 (segment (start 60.8884 53.497) (end 61.727 53.497) (width 0.25) (layer "F.Cu") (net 3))
 (segment (start 67.8774 64.931) (end 66.7952 64.931) (width 0.25) (layer "F.Cu") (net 3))
 (segment (start 60.071 53.312) (end 59.083 53.312) (width 0.25) (layer "F.Cu") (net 3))
 (segment (start 61.727 53.497) (end 61.727 54.3812) (width 0.25) (layer "F.Cu") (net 3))
 (segment (start 63.9452 64.976) (end 66.7502 64.976) (width 0.25) (layer "F.Cu") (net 3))
 (segment (start 61.6252 64.976) (end 61.6202 64.981) (width 0.25) (layer "F.Cu") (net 3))
 (via (at 60.6806 64.4398) (size 0.6) (drill 0.3) (layers "F.Cu" "B.Cu") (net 3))
 (via (at 56.7182 58.166) (size 0.6) (drill 0.3) (layers "F.Cu" "B.Cu") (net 3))
 (via (at 63.9452 64.976) (size 0.6) (drill 0.3) (layers "F.Cu" "B.Cu") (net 3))
 (via (at 59.0804 53.3146) (size 0.6) (drill 0.3) (layers "F.Cu" "B.Cu") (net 3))
 (via (at 68.453 61.4934) (size 0.6) (drill 0.3) (layers "F.Cu" "B.Cu") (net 3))
 (segment (start 63.9452 64.976) (end 64.9704 64.976) (width 0.25) (layer "B.Cu") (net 3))
 (segment (start 56.7182 54.8386) (end 58.2422 53.3146) (width 0.25) (layer "B.Cu") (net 3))
 (segment (start 63.915 64.9458) (end 63.9452 64.976) (width 0.25) (layer "B.Cu") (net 3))
 (segment (start 56.7182 60.4774) (end 60.6806 64.4398) (width 0.25) (layer "B.Cu") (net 3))
 (segment (start 58.2422 53.3146) (end 59.0804 53.3146) (width 0.25) (layer "B.Cu") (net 3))
 (segment (start 64.9704 64.976) (end 68.453 61.4934) (width 0.25) (layer "B.Cu") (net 3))
 (segment (start 56.7182 58.166) (end 56.7182 54.8386) (width 0.25) (layer "B.Cu") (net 3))
 (segment (start 56.7182 58.166) (end 56.7182 60.4774) (width 0.25) (layer "B.Cu") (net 3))
 (segment (start 60.6526 52.352) (end 60.8076 52.197) (width 0.25) (layer "F.Cu") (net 4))
 (segment (start 60.071 52.352) (end 60.6526 52.352) (width 0.25) (layer "F.Cu") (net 4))
 (segment (start 57.5564 53.1622) (end 58.3666 52.352) (width 0.25) (layer "F.Cu") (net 4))
 (segment (start 56.324 59.5) (end 57.5564 58.2676) (width 0.25) (layer "F.Cu") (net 4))
 (segment (start 64.8717 51.7397) (end 65.8622 51.7397) (width 0.25) (layer "F.Cu") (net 4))
 (segment (start 64.4144 52.197) (end 64.8717 51.7397) (width 0.25) (layer "F.Cu") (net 4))
 (segment (start 57.5564 56.3372) (end 57.5564 53.1622) (width 0.25) (layer "F.Cu") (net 4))
 (segment (start 57.5661 56.3275) (end 64.399584 56.3275) (width 0.25) (layer "F.Cu") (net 4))
 (segment (start 57.5564 58.2676) (end 57.5564 56.3372) (width 0.25) (layer "F.Cu") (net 4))
 (segment (start 63.627 52.197) (end 64.4144 52.197) (width 0.25) (layer "F.Cu") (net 4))
 (segment (start 57.5564 56.3372) (end 57.5661 56.3275) (width 0.25) (layer "F.Cu") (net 4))
 (segment (start 56.324 59.5) (end 54.98 59.5) (width 0.25) (layer "F.Cu") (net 4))
 (segment (start 58.3666 52.352) (end 60.071 52.352) (width 0.25) (layer "F.Cu") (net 4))
 (segment (start 64.399584 56.3275) (end 68.572084 60.5) (width 0.25) (layer "F.Cu") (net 4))
 (segment (start 68.572084 60.5) (end 70.42 60.5) (width 0.25) (layer "F.Cu") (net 4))
 (segment (start 61.727 52.197) (end 63.627 52.197) (width 0.25) (layer "F.Cu") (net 4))
 (segment (start 60.8076 52.197) (end 61.727 52.197) (width 0.25) (layer "F.Cu") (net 4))
 (segment (start 64.531 52.847) (end 63.627 52.847) (width 0.25) (layer "F.Cu") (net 10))
 (segment (start 65.8622 53.3147) (end 64.9987 53.3147) (width 0.25) (layer "F.Cu") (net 10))
 (segment (start 64.9987 53.3147) (end 64.531 52.847) (width 0.25) (layer "F.Cu") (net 10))
 (segment (start 57.24 61.5) (end 54.98 61.5) (width 0.25) (layer "F.Cu") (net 6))
 (segment (start 61.62 57.12) (end 57.24 61.5) (width 0.25) (layer "F.Cu") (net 6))
 (segment (start 68.453 58.49) (end 70.41 58.49) (width 0.25) (layer "F.Cu") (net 6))
 (segment (start 70.36 58.49) (end 70.37 58.5) (width 0.25) (layer "F.Cu") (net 6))
 (segment (start 70.41 58.49) (end 70.42 58.5) (width 0.25) (layer "F.Cu") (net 6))
 (segment (start 65.659 58.4708) (end 64.3082 57.12) (width 0.25) (layer "F.Cu") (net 6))
 (segment (start 70.31 58.49) (end 70.32 58.5) (width 0.25) (layer "F.Cu") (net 6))
 (segment (start 64.3082 57.12) (end 61.62 57.12) (width 0.25) (layer "F.Cu") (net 6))
 (via (at 68.453 58.49) (size 0.6) (drill 0.3) (layers "F.Cu" "B.Cu") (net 6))
 (via (at 65.659 58.4708) (size 0.6) (drill 0.3) (layers "F.Cu" "B.Cu") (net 6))
 (segment (start 68.453 58.49) (end 65.6782 58.49) (width 0.25) (layer "B.Cu") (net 6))
 (segment (start 65.6782 58.49) (end 65.659 58.4708) (width 0.25) (layer "B.Cu") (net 6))
 (segment (start 59.7916 57.2008) (end 59.7408 57.2008) (width 0.25) (layer "F.Cu") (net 5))
 (segment (start 68.472931 59.517669) (end 70.402331 59.517669) (width 0.25) (layer "F.Cu") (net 5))
 (segment (start 68.472931 59.517669) (end 68.4906 59.5) (width 0.25) (layer "F.Cu") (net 5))
 (segment (start 70.402331 59.517669) (end 70.42 59.5) (width 0.25) (layer "F.Cu") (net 5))
 (segment (start 59.7408 57.2008) (end 56.4416 60.5) (width 0.25) (layer "F.Cu") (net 5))
 (segment (start 56.4416 60.5) (end 54.98 60.5) (width 0.25) (layer "F.Cu") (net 5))
 (segment (start 68.472931 59.517669) (end 68.455262 59.5) (width 0.25) (layer "F.Cu") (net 5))
 (segment (start 70.352331 59.517669) (end 70.37 59.5) (width 0.25) (layer "F.Cu") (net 5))
 (via (at 59.7916 57.2008) (size 0.6) (drill 0.3) (layers "F.Cu" "B.Cu") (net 5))
 (via (at 68.472931 59.517669) (size 0.6) (drill 0.3) (layers "F.Cu" "B.Cu") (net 5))
 (segment (start 61.4492 57.2008) (end 59.7916 57.2008) (width 0.25) (layer "B.Cu") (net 5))
 (segment (start 68.472931 59.517669) (end 65.791469 59.517669) (width 0.25) (layer "B.Cu") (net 5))
 (segment (start 65.791469 59.517669) (end 63.4638 57.19) (width 0.25) (layer "B.Cu") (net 5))
 (segment (start 61.46 57.19) (end 61.4492 57.2008) (width 0.25) (layer "B.Cu") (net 5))
 (segment (start 63.4638 57.19) (end 61.46 57.19) (width 0.25) (layer "B.Cu") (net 5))
 (segment (start 63.627 54.4068) (end 63.1698 54.864) (width 0.25) (layer "F.Cu") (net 9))
 (segment (start 64.5202 65.881) (end 64.5202 66.081) (width 0.25) (layer "F.Cu") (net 9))
 (segment (start 62.8402 65.941) (end 62.8452 65.936) (width 0.25) (layer "F.Cu") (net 9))
 (segment (start 63.5452 65.936) (end 64.4652 65.936) (width 0.25) (layer "F.Cu") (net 9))
 (segment (start 61.6202 65.941) (end 60.4038 65.941) (width 0.25) (layer "F.Cu") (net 9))
 (segment (start 65.6082 68.5546) (end 65.1502 68.0966) (width 0.25) (layer "F.Cu") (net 9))
 (segment (start 58.55 65.1) (end 58.55 65.5858) (width 0.25) (layer "F.Cu") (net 9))
 (segment (start 62.8452 65.936) (end 63.5452 65.936) (width 0.25) (layer "F.Cu") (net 9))
 (segment (start 61.727 52.847) (end 62.1942 52.847) (width 0.25) (layer "F.Cu") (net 9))
 (segment (start 68.5546 68.5292) (end 65.6336 68.5292) (width 0.25) (layer "F.Cu") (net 9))
 (segment (start 65.1502 66.711) (end 65.1502 67.481) (width 0.25) (layer "F.Cu") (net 9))
 (segment (start 68.4754 54.6354) (end 68.83 54.99) (width 0.25) (layer "F.Cu") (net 9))
 (segment (start 63.627 53.497) (end 64.1396 53.497) (width 0.25) (layer "F.Cu") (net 9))
 (segment (start 65.278 54.6354) (end 68.4754 54.6354) (width 0.25) (layer "F.Cu") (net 9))
 (segment (start 62.1942 52.847) (end 62.8442 53.497) (width 0.25) (layer "F.Cu") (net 9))
 (segment (start 64.5202 66.081) (end 65.1502 66.711) (width 0.25) (layer "F.Cu") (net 9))
 (segment (start 61.6202 65.941) (end 62.8402 65.941) (width 0.25) (layer "F.Cu") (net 9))
 (segment (start 59.5628 65.1) (end 58.55 65.1) (width 0.25) (layer "F.Cu") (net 9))
 (segment (start 65.6336 68.5292) (end 65.6082 68.5546) (width 0.25) (layer "F.Cu") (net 9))
 (segment (start 63.627 53.497) (end 63.627 54.4068) (width 0.25) (layer "F.Cu") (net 9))
 (segment (start 64.1396 53.497) (end 65.278 54.6354) (width 0.25) (layer "F.Cu") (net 9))
 (segment (start 69.9008 67.183) (end 68.5546 68.5292) (width 0.25) (layer "F.Cu") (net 9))
 (segment (start 60.4038 65.941) (end 59.5628 65.1) (width 0.25) (layer "F.Cu") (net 9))
 (segment (start 69.9008 63.881) (end 69.9008 67.183) (width 0.25) (layer "F.Cu") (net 9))
 (segment (start 62.8442 53.497) (end 63.627 53.497) (width 0.25) (layer "F.Cu") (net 9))
 (segment (start 65.1502 68.0966) (end 65.1502 67.481) (width 0.25) (layer "F.Cu") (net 9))
 (segment (start 64.4652 65.936) (end 64.5202 65.881) (width 0.25) (layer "F.Cu") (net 9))
 (via (at 69.9008 63.881) (size 0.6) (drill 0.3) (layers "F.Cu" "B.Cu") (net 9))
 (via (at 68.83 54.99) (size 0.6) (drill 0.3) (layers "F.Cu" "B.Cu") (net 9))
 (segment (start 69.9008 56.0832) (end 68.83 55.0124) (width 0.25) (layer "B.Cu") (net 9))
 (segment (start 68.83 55.0124) (end 68.83 54.99) (width 0.25) (layer "B.Cu") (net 9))
 (segment (start 69.9008 63.881) (end 69.9008 56.0832) (width 0.25) (layer "B.Cu") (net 9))
 (segment (start 68.426 63.981) (end 68.4276 63.9826) (width 0.25) (layer "F.Cu") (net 1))
 (segment (start 66.7952 63.981) (end 66.7952 62.8252) (width 0.25) (layer "F.Cu") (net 1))
 (segment (start 66.7952 62.8252) (end 62.7 58.73) (width 0.25) (layer "F.Cu") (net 1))
 (segment (start 62.7 58.73) (end 63.02 58.73) (width 0.25) (layer "F.Cu") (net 1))
 (segment (start 66.7952 63.981) (end 68.426 63.981) (width 0.25) (layer "F.Cu") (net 1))
 (segment (start 57.6 62.56) (end 58.89 61.27) (width 0.25) (layer "F.Cu") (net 2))
 (segment (start 57.6 63.225) (end 57.6 62.56) (width 0.25) (layer "F.Cu") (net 2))
 (segment (start 58.89 61.27) (end 62.7 61.27) (width 0.25) (layer "F.Cu") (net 2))
 (segment (start 62.0058 63.225) (end 59.5 63.225) (width 0.25) (layer "F.Cu") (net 8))
 (segment (start 59.545 63.18) (end 59.5 63.225) (width 0.25) (layer "F.Cu") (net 8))
 (segment (start 64.5202 63.981) (end 62.7618 63.981) (width 0.25) (layer "F.Cu") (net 8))
 (segment (start 62.7618 63.981) (end 62.0058 63.225) (width 0.25) (layer "F.Cu") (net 8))
 (segment (start 66.7952 67.346) (end 66.6602 67.481) (width 0.25) (layer "F.Cu") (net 7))
 (segment (start 67.7164 67.3608) (end 68.4276 67.3608) (width 0.25) (layer "F.Cu") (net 7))
 (segment (start 66.7952 65.881) (end 66.7952 67.196) (width 0.25) (layer "F.Cu") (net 7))
 (segment (start 66.5226 67.481) (end 67.5962 67.481) (width 0.25) (layer "F.Cu") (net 7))
 (segment (start 66.5226 67.481) (end 66.1702 67.481) (width 0.25) (layer "F.Cu") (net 7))
 (segment (start 66.7952 67.196) (end 66.7952 67.346) (width 0.25) (layer "F.Cu") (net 7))
 (segment (start 66.6602 67.481) (end 66.5226 67.481) (width 0.25) (layer "F.Cu") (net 7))
 (segment (start 67.5962 67.481) (end 67.7164 67.3608) (width 0.25) (layer "F.Cu") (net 7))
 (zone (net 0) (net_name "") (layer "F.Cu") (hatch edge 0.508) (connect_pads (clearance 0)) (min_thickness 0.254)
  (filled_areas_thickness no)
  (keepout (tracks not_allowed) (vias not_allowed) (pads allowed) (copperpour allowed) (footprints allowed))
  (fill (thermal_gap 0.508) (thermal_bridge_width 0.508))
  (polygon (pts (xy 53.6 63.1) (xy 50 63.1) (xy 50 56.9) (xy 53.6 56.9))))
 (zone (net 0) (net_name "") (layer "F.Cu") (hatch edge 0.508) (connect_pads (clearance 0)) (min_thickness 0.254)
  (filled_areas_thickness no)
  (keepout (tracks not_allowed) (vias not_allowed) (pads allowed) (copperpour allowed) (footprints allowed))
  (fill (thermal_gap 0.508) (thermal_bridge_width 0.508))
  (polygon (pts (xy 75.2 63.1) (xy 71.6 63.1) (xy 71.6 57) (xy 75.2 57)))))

